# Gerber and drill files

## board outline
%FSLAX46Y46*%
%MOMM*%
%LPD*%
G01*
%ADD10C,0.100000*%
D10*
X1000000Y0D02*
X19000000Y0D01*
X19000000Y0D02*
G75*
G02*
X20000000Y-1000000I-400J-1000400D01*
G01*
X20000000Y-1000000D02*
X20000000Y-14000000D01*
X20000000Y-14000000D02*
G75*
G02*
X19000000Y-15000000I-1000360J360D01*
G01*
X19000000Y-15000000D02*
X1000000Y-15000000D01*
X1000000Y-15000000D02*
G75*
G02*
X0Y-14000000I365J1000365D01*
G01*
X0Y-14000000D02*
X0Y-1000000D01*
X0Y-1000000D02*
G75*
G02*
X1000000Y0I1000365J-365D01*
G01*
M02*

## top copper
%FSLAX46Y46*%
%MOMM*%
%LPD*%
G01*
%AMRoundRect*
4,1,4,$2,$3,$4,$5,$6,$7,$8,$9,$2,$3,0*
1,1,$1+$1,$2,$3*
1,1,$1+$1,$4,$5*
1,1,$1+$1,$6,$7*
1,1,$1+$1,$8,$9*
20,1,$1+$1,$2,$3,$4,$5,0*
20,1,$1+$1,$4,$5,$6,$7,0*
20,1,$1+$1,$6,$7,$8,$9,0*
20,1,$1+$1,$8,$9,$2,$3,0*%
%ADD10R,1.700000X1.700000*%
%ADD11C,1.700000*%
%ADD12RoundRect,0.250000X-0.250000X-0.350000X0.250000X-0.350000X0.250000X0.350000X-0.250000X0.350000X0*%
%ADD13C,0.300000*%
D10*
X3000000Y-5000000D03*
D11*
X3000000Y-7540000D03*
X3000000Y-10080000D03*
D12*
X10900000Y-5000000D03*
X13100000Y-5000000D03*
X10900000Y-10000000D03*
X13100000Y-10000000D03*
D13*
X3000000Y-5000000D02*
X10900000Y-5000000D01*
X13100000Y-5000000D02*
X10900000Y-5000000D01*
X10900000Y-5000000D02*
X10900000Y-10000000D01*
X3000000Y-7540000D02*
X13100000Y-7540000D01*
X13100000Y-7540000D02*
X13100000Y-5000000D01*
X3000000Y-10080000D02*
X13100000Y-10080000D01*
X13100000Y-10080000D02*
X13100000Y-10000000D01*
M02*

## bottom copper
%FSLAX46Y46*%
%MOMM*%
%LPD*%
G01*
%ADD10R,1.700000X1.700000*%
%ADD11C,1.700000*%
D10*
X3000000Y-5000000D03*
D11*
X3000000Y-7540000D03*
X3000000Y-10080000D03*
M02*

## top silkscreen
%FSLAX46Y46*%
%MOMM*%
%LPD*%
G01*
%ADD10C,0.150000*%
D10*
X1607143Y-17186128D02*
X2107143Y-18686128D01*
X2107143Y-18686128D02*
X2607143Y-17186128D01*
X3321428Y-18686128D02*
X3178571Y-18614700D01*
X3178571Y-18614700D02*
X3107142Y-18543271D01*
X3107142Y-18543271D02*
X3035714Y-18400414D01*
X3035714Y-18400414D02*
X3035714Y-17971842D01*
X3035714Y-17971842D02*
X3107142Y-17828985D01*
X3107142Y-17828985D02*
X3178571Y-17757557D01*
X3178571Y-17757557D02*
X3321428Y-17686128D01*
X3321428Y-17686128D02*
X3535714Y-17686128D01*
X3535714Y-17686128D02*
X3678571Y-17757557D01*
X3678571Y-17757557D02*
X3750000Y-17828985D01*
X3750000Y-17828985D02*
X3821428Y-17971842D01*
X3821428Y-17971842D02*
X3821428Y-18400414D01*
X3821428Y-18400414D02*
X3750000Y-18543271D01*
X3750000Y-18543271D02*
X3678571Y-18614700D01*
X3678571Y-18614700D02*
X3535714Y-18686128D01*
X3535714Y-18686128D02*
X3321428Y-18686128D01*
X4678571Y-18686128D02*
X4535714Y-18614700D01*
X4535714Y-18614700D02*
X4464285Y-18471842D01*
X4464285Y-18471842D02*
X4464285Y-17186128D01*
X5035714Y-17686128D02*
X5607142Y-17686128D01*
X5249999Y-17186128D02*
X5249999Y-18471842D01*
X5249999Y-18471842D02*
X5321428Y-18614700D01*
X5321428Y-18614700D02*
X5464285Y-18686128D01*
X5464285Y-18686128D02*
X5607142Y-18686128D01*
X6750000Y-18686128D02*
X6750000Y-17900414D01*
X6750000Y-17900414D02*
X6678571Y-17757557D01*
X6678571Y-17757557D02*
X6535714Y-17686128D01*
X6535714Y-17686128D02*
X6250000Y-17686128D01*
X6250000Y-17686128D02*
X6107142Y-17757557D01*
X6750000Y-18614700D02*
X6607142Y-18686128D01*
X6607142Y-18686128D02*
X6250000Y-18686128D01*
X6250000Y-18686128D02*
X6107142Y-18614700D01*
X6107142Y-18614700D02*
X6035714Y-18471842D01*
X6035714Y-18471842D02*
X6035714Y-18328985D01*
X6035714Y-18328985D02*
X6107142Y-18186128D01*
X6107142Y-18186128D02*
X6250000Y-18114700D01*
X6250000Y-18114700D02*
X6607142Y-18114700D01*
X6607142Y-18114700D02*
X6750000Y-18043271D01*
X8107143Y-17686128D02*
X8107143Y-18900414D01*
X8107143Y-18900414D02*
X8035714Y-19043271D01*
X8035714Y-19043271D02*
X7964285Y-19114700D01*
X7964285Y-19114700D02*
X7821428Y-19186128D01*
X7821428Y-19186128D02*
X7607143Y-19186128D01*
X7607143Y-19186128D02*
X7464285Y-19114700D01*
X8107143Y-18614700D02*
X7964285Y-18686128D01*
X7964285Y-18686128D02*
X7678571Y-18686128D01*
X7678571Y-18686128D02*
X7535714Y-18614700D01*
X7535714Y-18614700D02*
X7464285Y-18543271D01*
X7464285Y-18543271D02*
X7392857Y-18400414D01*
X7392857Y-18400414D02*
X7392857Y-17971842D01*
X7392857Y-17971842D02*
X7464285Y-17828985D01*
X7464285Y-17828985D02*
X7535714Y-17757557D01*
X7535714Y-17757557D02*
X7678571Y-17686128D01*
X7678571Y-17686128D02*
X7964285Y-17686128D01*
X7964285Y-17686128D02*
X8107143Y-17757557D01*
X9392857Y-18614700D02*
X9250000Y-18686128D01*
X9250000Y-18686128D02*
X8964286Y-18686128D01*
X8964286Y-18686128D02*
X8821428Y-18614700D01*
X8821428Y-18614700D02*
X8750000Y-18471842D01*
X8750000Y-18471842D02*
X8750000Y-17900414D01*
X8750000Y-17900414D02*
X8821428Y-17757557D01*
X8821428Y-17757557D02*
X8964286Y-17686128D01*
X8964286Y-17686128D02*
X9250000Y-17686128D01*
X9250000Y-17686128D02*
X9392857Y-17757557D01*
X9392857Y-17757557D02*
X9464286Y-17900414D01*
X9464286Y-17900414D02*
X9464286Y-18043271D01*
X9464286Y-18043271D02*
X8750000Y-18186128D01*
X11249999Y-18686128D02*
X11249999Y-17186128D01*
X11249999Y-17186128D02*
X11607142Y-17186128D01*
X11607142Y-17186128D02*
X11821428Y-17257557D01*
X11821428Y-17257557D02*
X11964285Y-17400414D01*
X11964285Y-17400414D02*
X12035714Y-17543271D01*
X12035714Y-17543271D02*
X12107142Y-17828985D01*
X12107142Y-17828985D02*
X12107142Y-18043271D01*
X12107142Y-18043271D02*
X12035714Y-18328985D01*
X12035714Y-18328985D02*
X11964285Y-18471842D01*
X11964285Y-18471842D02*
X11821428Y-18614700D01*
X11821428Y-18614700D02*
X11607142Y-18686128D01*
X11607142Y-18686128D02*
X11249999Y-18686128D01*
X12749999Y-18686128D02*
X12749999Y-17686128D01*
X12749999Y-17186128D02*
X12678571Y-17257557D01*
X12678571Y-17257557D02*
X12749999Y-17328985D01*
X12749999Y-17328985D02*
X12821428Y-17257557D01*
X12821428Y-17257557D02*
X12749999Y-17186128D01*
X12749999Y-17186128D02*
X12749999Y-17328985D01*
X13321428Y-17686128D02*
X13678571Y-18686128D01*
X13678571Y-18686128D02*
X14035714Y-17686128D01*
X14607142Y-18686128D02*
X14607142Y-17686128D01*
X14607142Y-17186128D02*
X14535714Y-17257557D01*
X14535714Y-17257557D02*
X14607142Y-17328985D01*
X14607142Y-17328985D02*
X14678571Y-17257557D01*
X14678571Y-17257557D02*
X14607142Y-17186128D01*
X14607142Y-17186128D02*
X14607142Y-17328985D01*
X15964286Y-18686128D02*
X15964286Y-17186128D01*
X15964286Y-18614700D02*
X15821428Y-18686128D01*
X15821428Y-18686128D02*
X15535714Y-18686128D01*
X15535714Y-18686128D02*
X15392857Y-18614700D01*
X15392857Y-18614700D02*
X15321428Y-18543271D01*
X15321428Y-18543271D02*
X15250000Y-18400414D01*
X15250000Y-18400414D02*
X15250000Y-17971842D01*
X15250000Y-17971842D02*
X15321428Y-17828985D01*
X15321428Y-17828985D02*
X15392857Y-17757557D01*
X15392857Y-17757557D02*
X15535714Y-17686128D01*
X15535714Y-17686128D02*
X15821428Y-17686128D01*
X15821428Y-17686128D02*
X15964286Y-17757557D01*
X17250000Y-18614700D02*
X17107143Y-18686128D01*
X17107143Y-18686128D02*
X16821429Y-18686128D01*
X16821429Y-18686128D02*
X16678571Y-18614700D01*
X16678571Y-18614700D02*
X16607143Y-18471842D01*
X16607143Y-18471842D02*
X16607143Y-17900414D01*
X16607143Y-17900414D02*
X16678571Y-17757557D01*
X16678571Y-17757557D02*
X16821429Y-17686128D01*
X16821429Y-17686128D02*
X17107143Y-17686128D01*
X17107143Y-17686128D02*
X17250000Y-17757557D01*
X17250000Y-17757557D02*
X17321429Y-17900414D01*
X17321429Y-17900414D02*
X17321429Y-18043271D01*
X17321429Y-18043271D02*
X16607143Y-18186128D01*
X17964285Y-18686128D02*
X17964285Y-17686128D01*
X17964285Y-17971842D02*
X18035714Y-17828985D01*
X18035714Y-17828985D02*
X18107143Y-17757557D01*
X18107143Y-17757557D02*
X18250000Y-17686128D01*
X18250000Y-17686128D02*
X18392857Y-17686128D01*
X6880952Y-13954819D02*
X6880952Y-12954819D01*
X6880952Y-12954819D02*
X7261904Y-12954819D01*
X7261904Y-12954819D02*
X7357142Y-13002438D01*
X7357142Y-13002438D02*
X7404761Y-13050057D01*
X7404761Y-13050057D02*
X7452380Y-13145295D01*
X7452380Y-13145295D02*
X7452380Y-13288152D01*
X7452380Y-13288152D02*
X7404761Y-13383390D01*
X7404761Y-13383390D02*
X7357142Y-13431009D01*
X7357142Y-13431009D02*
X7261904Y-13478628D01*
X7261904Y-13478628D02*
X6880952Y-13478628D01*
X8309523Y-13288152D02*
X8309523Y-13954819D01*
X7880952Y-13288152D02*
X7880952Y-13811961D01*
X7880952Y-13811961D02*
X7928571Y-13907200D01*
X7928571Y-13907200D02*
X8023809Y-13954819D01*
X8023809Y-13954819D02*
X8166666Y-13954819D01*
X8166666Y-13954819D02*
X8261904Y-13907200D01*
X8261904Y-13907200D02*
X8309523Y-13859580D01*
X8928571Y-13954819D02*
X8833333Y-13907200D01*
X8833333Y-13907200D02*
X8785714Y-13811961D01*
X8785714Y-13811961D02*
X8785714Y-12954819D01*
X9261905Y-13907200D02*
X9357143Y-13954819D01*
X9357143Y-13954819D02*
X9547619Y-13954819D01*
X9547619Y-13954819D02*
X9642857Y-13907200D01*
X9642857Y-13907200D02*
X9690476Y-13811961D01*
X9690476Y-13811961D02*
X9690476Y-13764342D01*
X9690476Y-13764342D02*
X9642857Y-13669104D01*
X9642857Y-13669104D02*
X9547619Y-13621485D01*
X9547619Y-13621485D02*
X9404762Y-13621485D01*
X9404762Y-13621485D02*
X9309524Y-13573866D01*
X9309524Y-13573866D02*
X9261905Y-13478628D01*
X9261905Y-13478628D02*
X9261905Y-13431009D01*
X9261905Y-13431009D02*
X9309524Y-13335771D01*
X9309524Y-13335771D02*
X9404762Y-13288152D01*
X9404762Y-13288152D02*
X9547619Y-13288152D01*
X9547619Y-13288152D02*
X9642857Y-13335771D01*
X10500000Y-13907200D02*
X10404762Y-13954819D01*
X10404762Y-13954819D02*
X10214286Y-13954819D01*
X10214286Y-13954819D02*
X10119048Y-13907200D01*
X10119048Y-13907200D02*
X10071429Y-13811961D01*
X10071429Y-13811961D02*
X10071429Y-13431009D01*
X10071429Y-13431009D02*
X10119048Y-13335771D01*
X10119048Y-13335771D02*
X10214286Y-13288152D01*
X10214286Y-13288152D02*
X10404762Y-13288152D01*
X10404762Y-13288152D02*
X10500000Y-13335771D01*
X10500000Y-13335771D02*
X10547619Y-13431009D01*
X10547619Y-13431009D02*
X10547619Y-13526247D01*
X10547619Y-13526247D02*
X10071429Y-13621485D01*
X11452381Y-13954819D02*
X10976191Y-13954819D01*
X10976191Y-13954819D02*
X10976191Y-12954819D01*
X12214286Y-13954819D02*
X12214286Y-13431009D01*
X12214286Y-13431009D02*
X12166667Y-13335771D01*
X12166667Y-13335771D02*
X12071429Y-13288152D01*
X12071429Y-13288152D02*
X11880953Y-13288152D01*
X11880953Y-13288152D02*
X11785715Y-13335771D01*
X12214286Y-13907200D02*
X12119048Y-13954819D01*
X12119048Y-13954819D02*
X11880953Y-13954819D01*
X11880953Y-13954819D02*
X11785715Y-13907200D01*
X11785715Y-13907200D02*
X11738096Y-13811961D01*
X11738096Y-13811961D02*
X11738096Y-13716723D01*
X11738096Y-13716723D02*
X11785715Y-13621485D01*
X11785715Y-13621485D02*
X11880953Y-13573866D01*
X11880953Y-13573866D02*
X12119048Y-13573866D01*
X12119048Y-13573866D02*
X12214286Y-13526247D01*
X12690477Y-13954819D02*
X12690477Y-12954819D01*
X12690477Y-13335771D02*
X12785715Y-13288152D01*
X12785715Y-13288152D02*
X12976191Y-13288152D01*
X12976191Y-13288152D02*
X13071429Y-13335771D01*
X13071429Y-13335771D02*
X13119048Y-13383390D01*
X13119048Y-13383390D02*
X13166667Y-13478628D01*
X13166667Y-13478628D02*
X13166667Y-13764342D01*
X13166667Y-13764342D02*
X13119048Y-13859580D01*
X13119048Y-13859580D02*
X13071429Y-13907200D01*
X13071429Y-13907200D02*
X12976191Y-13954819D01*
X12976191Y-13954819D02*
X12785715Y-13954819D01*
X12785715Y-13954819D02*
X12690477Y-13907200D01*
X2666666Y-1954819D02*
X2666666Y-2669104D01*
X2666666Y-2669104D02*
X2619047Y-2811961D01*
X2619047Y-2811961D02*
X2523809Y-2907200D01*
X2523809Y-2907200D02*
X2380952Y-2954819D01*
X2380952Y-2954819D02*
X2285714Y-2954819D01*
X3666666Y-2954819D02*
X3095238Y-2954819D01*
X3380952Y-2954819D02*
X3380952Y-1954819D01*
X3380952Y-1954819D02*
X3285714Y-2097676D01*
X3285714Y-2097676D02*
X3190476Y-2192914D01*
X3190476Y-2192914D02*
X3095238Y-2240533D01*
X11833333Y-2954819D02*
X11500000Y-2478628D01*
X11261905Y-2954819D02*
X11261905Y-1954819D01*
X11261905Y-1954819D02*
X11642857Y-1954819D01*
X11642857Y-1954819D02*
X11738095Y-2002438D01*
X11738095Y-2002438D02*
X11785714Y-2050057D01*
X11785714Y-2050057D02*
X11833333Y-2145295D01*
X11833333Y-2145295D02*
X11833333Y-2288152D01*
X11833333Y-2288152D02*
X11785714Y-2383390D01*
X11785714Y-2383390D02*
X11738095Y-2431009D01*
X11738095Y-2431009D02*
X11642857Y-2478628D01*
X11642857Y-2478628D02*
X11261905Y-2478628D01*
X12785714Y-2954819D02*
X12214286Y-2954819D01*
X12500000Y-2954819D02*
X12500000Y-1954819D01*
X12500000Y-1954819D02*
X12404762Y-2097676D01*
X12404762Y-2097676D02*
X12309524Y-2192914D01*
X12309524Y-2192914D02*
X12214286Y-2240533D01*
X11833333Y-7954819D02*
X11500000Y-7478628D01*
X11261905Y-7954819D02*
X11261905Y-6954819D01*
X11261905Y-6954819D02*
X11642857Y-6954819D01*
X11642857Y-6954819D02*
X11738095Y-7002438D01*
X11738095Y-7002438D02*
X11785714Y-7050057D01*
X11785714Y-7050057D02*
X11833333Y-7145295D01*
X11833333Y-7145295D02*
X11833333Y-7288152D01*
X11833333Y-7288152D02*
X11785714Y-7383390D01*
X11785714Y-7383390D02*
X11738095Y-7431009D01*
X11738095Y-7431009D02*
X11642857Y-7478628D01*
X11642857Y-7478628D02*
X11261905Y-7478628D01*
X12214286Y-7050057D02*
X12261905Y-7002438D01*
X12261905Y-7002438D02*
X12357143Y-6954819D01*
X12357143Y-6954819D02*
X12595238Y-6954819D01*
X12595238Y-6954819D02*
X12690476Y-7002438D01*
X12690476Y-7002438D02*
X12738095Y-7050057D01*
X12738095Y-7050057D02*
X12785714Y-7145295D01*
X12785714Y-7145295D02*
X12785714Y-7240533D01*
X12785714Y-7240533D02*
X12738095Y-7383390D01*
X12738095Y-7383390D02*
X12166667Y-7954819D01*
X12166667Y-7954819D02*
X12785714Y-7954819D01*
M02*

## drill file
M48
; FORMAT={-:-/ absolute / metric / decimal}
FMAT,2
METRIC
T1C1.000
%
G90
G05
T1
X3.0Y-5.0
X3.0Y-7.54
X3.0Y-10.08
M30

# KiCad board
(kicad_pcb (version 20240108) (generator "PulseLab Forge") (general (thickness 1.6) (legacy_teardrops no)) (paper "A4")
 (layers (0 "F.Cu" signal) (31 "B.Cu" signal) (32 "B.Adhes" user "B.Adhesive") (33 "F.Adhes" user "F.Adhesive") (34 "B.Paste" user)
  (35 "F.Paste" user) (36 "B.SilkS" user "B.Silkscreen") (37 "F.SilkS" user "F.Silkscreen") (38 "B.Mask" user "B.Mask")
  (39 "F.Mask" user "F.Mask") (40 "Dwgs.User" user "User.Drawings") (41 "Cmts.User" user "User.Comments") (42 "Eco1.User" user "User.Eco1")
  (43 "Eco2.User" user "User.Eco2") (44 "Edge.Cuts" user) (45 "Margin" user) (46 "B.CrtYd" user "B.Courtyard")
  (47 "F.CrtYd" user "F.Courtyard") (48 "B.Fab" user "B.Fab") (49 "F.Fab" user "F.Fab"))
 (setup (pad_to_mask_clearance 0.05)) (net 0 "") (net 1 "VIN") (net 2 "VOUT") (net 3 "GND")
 (gr_line (start 1.000 0.000) (end 19.000 0.000) (layer "Edge.Cuts") (stroke (width 0.1)))
 (gr_arc (start 19.000 0.000) (mid 19.707 0.293) (end 20.000 1.000) (layer "Edge.Cuts") (stroke (width 0.1)))
 (gr_line (start 20.000 1.000) (end 20.000 14.000) (layer "Edge.Cuts") (stroke (width 0.1)))
 (gr_arc (start 20.000 14.000) (mid 19.707 14.707) (end 19.000 15.000) (layer "Edge.Cuts") (stroke (width 0.1)))
 (gr_line (start 19.000 15.000) (end 1.000 15.000) (layer "Edge.Cuts") (stroke (width 0.1)))
 (gr_arc (start 1.000 15.000) (mid 0.293 14.707) (end 0.000 14.000) (layer "Edge.Cuts") (stroke (width 0.1)))
 (gr_line (start 0.000 14.000) (end 0.000 1.000) (layer "Edge.Cuts") (stroke (width 0.1)))
 (gr_arc (start 0.000 1.000) (mid 0.293 0.293) (end 1.000 0.000) (layer "Edge.Cuts") (stroke (width 0.1)))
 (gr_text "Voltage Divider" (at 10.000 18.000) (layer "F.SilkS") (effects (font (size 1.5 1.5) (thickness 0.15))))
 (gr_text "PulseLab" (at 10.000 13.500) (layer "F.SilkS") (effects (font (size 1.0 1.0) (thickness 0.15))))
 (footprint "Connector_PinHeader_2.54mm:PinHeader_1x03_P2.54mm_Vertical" (layer "F.Cu") (at 3.0000 5.0000)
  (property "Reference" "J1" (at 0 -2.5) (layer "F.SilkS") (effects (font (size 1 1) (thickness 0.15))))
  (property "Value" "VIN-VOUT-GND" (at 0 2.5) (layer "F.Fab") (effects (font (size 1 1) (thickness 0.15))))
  (pad "1" thru_hole rect (at 0.0000 0.0000) (size 1.7000 1.7000) (drill 1.0) (layers "*.Cu" "*.Mask") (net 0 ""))
  (pad "2" thru_hole circle (at 0.0000 2.5400) (size 1.7000 1.7000) (drill 1.0) (layers "*.Cu" "*.Mask") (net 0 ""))
  (pad "3" thru_hole circle (at 0.0000 5.0800) (size 1.7000 1.7000) (drill 1.0) (layers "*.Cu" "*.Mask") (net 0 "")))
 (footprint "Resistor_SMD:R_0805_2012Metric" (layer "F.Cu") (at 12.0000 5.0000)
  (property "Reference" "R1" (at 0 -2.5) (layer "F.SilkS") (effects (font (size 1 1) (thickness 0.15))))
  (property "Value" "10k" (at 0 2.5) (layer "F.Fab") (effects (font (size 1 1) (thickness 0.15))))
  (pad "1" smd roundrect (at -1.1000 0.0000) (size 1.0000 1.2000) (layers "F.Cu" "F.Paste" "F.Mask") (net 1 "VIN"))
  (pad "2" smd roundrect (at 1.1000 0.0000) (size 1.0000 1.2000) (layers "F.Cu" "F.Paste" "F.Mask") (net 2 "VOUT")))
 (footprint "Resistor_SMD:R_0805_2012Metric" (layer "F.Cu") (at 12.0000 10.0000)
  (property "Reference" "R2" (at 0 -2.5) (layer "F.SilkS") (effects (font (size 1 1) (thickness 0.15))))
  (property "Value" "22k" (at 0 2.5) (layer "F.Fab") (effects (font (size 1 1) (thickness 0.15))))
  (pad "1" smd roundrect (at -1.1000 0.0000) (size 1.0000 1.2000) (layers "F.Cu" "F.Paste" "F.Mask") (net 2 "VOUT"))
  (pad "2" smd roundrect (at 1.1000 0.0000) (size 1.0000 1.2000) (layers "F.Cu" "F.Paste" "F.Mask") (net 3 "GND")))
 (segment (start 3.0000 5.0000) (end 10.9000 5.0000) (width 0.3000) (layer "F.Cu") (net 1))
 (segment (start 13.1000 5.0000) (end 10.9000 5.0000) (width 0.3000) (layer "F.Cu") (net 2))
 (segment (start 10.9000 5.0000) (end 10.9000 10.0000) (width 0.3000) (layer "F.Cu") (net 2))
 (segment (start 3.0000 7.5400) (end 13.1000 7.5400) (width 0.3000) (layer "F.Cu") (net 2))
 (segment (start 13.1000 7.5400) (end 13.1000 5.0000) (width 0.3000) (layer "F.Cu") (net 2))
 (segment (start 3.0000 10.0800) (end 13.1000 10.0800) (width 0.3000) (layer "F.Cu") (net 3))
 (segment (start 13.1000 10.0800) (end 13.1000 10.0000) (width 0.3000) (layer "F.Cu") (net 3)))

